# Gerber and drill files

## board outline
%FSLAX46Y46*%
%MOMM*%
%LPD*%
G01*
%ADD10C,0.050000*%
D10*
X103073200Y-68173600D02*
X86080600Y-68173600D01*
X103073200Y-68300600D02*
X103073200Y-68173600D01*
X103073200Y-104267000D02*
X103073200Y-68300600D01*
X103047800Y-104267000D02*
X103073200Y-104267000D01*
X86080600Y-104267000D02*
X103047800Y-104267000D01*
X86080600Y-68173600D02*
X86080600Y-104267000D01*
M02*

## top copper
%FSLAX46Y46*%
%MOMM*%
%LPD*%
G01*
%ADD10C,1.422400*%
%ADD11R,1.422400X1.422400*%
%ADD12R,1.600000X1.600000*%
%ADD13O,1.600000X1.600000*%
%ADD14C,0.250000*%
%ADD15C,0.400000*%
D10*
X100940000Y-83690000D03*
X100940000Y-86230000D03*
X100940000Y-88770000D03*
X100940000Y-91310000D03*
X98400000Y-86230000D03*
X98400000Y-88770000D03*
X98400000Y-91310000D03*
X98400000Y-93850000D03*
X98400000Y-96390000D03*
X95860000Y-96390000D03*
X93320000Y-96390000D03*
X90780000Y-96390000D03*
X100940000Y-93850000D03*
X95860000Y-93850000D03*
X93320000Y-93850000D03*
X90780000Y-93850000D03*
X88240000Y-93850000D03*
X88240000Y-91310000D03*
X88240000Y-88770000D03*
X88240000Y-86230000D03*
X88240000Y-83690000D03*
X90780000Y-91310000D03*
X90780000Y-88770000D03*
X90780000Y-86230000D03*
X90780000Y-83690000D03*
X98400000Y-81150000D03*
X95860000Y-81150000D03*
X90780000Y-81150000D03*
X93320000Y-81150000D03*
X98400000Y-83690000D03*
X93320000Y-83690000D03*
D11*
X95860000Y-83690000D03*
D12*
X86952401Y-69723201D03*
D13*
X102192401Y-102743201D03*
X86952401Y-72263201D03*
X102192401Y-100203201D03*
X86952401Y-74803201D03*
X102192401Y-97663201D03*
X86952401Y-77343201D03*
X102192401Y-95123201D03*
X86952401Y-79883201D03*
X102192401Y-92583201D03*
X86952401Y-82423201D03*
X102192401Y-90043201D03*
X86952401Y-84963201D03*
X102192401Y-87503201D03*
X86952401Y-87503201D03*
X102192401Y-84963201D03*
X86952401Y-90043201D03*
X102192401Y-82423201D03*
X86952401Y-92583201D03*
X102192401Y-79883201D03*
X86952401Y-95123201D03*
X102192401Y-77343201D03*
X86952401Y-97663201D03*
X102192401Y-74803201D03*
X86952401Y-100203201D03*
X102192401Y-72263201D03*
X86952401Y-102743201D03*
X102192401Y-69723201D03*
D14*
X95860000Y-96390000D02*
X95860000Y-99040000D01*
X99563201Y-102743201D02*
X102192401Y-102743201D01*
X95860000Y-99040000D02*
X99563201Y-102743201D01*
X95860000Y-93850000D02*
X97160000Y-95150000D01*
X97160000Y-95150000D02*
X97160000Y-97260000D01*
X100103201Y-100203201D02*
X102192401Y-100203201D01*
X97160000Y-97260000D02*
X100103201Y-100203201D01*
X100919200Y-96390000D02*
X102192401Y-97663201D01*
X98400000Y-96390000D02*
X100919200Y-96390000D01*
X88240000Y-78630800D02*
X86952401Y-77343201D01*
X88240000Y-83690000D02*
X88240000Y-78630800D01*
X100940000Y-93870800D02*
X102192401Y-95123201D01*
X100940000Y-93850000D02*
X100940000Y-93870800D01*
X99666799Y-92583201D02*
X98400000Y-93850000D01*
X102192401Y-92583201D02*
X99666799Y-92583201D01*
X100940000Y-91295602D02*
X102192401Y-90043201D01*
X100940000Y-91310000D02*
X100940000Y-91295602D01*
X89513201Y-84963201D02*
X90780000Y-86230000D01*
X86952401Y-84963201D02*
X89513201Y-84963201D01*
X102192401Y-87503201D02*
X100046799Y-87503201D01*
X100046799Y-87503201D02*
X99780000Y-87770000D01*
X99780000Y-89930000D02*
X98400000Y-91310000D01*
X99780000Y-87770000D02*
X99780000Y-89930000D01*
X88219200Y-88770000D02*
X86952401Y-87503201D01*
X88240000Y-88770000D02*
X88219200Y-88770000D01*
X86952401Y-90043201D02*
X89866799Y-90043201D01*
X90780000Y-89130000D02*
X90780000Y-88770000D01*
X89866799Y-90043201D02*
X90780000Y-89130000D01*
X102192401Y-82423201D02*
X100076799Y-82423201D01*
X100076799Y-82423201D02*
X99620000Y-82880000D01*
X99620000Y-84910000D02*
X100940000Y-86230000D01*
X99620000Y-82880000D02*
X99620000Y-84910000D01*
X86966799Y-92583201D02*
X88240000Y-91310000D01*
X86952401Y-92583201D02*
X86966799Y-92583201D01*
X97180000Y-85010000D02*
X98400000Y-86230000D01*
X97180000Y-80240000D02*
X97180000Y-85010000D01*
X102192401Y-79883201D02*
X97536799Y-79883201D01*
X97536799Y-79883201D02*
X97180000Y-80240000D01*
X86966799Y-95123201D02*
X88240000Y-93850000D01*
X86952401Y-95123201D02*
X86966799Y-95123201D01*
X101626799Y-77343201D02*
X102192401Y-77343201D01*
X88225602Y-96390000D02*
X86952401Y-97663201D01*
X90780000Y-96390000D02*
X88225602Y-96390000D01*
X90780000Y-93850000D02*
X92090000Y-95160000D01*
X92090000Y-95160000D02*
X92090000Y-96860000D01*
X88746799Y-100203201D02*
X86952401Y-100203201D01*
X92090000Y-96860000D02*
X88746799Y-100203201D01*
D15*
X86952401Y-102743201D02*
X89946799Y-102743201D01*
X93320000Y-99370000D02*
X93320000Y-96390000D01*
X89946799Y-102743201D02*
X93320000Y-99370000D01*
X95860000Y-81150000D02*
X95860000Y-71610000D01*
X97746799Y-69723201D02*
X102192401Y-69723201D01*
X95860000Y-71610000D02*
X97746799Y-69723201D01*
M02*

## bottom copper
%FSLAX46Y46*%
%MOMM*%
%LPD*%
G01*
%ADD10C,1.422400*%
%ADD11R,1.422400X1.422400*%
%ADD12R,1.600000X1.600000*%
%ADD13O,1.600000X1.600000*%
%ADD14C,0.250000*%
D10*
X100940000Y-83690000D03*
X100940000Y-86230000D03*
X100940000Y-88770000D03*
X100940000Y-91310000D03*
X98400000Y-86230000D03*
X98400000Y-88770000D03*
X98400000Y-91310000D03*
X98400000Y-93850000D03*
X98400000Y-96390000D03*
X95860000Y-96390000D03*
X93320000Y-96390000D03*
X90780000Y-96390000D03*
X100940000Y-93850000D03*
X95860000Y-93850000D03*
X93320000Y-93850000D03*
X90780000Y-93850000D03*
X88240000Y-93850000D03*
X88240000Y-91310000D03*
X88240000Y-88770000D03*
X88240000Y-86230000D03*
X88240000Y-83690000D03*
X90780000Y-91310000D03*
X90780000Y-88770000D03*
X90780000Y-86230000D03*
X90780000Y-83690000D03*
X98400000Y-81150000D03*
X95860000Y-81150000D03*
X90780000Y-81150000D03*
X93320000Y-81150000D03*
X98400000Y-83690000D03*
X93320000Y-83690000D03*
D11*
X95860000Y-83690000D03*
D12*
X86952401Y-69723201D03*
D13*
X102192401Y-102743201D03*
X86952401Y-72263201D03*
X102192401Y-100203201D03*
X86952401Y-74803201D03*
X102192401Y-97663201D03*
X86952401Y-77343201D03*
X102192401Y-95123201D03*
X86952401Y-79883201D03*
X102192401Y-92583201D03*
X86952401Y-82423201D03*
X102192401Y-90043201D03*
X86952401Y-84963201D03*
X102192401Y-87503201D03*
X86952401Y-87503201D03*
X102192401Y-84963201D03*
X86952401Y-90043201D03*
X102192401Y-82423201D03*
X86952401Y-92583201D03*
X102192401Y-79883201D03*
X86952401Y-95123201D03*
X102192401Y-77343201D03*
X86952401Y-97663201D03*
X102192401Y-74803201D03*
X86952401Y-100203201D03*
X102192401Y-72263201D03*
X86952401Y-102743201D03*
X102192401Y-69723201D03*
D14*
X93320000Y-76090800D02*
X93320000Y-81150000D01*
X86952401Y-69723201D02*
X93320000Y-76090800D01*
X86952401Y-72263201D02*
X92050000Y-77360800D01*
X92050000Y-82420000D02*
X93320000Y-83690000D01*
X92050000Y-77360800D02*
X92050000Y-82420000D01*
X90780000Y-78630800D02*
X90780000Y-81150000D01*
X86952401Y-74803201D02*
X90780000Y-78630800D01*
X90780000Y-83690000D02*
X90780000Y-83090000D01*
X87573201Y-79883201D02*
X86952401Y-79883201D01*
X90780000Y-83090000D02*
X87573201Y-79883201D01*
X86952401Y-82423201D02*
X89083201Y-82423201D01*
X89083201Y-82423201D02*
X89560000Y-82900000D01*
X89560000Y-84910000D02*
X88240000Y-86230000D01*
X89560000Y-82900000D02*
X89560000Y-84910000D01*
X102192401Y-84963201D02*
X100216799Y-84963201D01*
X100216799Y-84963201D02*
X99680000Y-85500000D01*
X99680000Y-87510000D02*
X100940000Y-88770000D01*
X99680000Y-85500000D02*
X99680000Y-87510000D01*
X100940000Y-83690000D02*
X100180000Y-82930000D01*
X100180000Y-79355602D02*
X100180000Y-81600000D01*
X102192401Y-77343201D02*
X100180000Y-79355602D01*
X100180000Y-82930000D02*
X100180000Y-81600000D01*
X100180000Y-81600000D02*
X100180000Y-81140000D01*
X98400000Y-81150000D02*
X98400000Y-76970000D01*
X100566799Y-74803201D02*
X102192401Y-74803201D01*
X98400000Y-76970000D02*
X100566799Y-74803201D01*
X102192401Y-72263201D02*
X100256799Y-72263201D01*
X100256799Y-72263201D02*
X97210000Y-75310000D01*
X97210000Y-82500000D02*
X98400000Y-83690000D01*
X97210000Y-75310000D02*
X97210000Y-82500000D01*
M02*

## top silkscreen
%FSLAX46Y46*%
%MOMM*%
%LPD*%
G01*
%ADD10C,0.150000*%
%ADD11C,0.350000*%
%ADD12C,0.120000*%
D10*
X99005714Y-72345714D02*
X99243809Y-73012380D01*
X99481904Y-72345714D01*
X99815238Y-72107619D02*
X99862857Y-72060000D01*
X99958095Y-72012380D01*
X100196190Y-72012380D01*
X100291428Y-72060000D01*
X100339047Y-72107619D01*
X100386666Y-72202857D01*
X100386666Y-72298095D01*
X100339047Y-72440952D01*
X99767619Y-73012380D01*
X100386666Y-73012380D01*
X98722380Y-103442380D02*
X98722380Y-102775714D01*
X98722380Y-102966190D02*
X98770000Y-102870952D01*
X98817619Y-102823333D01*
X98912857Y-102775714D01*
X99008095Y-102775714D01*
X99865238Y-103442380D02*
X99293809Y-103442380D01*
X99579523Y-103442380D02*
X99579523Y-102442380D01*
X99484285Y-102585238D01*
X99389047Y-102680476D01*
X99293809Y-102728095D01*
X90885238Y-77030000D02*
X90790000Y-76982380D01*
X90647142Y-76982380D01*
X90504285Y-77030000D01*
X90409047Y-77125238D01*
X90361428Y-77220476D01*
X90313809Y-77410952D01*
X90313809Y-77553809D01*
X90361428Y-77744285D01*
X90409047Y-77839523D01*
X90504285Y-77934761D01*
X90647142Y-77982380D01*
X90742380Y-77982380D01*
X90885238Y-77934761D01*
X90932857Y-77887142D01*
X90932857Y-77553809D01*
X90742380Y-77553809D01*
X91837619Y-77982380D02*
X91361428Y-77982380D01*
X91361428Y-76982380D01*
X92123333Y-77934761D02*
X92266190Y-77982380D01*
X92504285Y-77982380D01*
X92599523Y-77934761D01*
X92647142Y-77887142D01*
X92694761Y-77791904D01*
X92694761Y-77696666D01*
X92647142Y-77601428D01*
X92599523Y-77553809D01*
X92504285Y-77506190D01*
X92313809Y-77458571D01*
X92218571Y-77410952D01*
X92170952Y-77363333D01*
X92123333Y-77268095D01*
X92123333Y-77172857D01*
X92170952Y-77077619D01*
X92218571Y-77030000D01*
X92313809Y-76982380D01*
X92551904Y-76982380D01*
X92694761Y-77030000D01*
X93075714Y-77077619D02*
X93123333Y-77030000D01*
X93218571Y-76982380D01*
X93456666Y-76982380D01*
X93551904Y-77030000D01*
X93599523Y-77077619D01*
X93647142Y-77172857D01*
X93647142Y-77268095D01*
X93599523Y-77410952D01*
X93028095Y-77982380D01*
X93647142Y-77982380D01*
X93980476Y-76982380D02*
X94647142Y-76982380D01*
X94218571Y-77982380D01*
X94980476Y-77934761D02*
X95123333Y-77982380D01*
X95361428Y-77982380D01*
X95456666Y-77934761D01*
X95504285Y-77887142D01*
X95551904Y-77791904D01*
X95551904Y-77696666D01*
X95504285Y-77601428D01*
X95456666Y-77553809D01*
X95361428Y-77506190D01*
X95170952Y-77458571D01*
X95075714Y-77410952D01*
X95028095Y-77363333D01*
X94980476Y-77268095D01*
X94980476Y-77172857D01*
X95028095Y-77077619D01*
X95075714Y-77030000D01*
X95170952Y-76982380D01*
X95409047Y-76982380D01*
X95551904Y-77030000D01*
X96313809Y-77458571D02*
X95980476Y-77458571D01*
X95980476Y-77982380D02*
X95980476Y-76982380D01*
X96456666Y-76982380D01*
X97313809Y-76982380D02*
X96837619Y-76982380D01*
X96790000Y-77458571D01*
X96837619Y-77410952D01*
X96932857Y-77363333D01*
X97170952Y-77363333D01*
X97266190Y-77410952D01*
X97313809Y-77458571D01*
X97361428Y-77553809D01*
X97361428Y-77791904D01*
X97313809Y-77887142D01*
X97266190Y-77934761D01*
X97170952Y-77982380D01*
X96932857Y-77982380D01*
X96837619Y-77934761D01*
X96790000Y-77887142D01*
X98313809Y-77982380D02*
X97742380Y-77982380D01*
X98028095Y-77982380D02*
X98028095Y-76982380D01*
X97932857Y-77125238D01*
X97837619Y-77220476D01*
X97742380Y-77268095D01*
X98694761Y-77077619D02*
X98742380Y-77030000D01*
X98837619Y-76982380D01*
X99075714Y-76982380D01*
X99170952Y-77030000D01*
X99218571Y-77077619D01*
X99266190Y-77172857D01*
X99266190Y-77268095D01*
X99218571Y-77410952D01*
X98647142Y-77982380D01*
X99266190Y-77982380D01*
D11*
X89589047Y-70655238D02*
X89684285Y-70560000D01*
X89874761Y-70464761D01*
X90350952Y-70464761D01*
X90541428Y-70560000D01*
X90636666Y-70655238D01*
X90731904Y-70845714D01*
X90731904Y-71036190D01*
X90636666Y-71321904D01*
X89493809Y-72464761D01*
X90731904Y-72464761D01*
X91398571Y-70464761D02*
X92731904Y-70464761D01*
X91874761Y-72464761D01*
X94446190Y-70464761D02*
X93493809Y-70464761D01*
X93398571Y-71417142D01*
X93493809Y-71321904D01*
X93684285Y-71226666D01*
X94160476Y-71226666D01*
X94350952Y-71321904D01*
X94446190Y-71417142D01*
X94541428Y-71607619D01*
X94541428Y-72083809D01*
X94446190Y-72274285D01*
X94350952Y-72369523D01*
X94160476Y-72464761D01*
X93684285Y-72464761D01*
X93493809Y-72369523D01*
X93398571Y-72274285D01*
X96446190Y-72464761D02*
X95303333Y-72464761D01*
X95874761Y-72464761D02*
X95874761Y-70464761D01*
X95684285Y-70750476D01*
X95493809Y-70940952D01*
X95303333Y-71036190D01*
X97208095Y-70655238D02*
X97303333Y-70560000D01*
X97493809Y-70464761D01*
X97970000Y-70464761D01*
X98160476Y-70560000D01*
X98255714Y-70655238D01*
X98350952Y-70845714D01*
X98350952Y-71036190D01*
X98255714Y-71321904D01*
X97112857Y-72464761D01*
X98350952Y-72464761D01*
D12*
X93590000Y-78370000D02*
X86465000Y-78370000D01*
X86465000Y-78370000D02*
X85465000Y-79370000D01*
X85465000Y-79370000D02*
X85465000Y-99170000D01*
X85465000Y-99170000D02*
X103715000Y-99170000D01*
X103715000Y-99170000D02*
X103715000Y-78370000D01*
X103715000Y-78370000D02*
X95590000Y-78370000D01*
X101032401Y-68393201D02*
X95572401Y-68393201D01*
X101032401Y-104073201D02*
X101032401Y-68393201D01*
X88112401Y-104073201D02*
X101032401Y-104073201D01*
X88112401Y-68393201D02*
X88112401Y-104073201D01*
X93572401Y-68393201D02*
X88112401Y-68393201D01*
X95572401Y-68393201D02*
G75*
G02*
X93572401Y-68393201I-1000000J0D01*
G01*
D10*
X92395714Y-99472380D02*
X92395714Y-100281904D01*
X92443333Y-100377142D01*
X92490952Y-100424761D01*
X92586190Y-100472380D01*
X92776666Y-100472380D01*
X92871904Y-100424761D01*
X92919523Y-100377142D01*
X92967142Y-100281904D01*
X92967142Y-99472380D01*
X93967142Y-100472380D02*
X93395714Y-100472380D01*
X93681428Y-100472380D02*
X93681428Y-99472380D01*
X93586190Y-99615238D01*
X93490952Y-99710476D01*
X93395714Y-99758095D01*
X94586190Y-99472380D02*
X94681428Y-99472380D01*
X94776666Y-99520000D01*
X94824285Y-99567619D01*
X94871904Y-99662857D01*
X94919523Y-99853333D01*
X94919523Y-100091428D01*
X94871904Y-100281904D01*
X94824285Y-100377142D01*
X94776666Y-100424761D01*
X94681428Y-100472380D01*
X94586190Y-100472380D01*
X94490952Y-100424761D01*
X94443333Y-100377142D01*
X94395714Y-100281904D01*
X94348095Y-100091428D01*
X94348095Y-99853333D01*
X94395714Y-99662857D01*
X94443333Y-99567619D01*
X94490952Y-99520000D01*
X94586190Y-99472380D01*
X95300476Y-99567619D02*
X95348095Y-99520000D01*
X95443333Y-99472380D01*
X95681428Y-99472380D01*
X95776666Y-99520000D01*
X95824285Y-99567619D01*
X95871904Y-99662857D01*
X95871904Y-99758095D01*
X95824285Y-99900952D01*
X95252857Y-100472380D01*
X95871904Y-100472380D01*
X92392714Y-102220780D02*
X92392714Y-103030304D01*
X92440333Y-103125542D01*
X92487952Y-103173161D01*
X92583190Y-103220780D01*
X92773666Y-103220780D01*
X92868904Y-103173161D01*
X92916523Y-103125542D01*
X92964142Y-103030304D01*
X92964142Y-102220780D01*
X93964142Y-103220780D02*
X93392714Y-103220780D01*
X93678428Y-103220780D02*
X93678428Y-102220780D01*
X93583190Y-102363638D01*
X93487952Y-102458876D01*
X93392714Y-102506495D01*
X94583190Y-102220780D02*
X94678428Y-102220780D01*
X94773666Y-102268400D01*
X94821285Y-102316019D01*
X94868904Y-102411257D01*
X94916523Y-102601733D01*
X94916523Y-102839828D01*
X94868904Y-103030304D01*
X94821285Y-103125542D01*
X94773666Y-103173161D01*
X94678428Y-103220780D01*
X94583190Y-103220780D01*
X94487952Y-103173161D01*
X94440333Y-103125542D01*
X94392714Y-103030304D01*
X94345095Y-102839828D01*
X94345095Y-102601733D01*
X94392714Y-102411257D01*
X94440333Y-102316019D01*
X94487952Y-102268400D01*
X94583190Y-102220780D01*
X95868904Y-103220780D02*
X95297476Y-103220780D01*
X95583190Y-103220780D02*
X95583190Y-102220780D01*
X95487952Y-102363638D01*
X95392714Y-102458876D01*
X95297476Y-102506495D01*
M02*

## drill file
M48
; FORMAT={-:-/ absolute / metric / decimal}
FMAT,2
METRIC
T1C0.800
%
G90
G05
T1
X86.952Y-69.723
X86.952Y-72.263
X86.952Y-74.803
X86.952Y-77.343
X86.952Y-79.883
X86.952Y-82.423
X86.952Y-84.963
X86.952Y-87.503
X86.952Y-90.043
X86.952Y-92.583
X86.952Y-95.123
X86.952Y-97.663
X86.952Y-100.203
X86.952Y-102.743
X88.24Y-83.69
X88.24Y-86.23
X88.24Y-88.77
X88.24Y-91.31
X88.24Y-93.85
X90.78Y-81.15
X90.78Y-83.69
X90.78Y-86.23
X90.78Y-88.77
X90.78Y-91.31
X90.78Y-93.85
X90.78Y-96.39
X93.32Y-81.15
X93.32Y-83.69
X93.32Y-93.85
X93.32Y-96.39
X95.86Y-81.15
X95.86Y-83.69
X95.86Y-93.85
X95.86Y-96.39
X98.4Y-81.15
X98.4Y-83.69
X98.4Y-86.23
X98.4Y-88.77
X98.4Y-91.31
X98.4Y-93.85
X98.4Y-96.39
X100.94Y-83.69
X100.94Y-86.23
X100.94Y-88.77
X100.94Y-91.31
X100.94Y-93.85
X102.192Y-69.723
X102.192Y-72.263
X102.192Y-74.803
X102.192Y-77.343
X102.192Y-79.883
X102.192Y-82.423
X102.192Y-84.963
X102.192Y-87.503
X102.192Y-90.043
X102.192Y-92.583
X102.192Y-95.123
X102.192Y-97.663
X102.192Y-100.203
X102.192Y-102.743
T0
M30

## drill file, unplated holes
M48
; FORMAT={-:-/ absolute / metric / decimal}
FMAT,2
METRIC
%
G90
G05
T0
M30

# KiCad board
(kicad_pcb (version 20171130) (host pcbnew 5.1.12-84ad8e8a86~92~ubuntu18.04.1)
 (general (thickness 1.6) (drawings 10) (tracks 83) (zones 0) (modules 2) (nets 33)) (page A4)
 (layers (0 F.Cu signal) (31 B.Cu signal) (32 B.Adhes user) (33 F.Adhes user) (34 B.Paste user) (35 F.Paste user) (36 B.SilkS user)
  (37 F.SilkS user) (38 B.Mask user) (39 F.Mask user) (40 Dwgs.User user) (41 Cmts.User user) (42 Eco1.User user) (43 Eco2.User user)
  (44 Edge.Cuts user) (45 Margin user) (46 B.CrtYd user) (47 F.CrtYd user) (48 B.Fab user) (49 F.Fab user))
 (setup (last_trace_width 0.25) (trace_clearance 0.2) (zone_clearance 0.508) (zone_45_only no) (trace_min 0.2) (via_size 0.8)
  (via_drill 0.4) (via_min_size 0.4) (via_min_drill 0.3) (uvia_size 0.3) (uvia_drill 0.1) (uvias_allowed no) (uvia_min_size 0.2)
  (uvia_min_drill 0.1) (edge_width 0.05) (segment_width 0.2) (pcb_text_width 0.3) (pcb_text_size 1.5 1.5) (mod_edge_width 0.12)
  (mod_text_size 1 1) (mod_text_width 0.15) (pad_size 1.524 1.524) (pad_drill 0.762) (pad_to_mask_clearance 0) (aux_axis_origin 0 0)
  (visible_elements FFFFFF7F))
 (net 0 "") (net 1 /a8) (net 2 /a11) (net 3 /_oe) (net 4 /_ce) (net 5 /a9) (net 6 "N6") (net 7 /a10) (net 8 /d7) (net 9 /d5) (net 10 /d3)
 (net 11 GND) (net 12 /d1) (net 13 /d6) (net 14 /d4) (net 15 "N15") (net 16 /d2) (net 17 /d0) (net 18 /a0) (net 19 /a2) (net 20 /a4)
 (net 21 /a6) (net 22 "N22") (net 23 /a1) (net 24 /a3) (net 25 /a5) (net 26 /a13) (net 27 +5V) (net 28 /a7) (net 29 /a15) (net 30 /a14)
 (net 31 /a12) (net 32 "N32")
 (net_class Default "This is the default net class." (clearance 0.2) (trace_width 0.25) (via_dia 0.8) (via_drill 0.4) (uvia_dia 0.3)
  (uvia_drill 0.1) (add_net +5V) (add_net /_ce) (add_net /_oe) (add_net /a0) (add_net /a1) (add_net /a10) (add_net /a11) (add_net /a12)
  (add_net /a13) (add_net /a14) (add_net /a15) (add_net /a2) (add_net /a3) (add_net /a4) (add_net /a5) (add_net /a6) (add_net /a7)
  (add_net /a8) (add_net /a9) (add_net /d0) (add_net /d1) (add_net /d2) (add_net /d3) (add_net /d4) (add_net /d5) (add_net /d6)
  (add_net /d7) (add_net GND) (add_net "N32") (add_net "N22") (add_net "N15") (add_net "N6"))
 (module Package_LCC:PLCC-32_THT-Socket (layer F.Cu) (at 95.86 83.69)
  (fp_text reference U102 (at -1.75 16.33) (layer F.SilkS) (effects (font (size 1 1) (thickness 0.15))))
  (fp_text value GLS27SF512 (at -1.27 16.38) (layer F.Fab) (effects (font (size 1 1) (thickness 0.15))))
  (fp_line (start -2.27 -5.32) (end -9.395 -5.32) (layer F.SilkS) (width 0.12))
  (fp_line (start -9.395 -5.32) (end -10.395 -4.32) (layer F.SilkS) (width 0.12))
  (fp_line (start -10.395 -4.32) (end -10.395 15.48) (layer F.SilkS) (width 0.12))
  (fp_line (start -10.395 15.48) (end 7.855 15.48) (layer F.SilkS) (width 0.12))
  (fp_line (start 7.855 15.48) (end 7.855 -5.32) (layer F.SilkS) (width 0.12))
  (fp_line (start 7.855 -5.32) (end -0.27 -5.32) (layer F.SilkS) (width 0.12))
  (pad 29 thru_hole circle (at 5.08 0) (size 1.4224 1.4224) (drill 0.8) (layers *.Cu *.Mask) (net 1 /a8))
  (pad 27 thru_hole circle (at 5.08 2.54) (size 1.4224 1.4224) (drill 0.8) (layers *.Cu *.Mask) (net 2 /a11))
  (pad 25 thru_hole circle (at 5.08 5.08) (size 1.4224 1.4224) (drill 0.8) (layers *.Cu *.Mask) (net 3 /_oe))
  (pad 23 thru_hole circle (at 5.08 7.62) (size 1.4224 1.4224) (drill 0.8) (layers *.Cu *.Mask) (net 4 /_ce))
  (pad 28 thru_hole circle (at 2.54 2.54) (size 1.4224 1.4224) (drill 0.8) (layers *.Cu *.Mask) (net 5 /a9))
  (pad 26 thru_hole circle (at 2.54 5.08) (size 1.4224 1.4224) (drill 0.8) (layers *.Cu *.Mask) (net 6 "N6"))
  (pad 24 thru_hole circle (at 2.54 7.62) (size 1.4224 1.4224) (drill 0.8) (layers *.Cu *.Mask) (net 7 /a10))
  (pad 22 thru_hole circle (at 2.54 10.16) (size 1.4224 1.4224) (drill 0.8) (layers *.Cu *.Mask) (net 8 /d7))
  (pad 20 thru_hole circle (at 2.54 12.7) (size 1.4224 1.4224) (drill 0.8) (layers *.Cu *.Mask) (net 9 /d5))
  (pad 18 thru_hole circle (at 0 12.7) (size 1.4224 1.4224) (drill 0.8) (layers *.Cu *.Mask) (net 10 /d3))
  (pad 16 thru_hole circle (at -2.54 12.7) (size 1.4224 1.4224) (drill 0.8) (layers *.Cu *.Mask) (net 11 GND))
  (pad 14 thru_hole circle (at -5.08 12.7) (size 1.4224 1.4224) (drill 0.8) (layers *.Cu *.Mask) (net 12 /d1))
  (pad 21 thru_hole circle (at 5.08 10.16) (size 1.4224 1.4224) (drill 0.8) (layers *.Cu *.Mask) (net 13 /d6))
  (pad 19 thru_hole circle (at 0 10.16) (size 1.4224 1.4224) (drill 0.8) (layers *.Cu *.Mask) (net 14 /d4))
  (pad 17 thru_hole circle (at -2.54 10.16) (size 1.4224 1.4224) (drill 0.8) (layers *.Cu *.Mask) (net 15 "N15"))
  (pad 15 thru_hole circle (at -5.08 10.16) (size 1.4224 1.4224) (drill 0.8) (layers *.Cu *.Mask) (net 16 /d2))
  (pad 13 thru_hole circle (at -7.62 10.16) (size 1.4224 1.4224) (drill 0.8) (layers *.Cu *.Mask) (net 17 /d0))
  (pad 11 thru_hole circle (at -7.62 7.62) (size 1.4224 1.4224) (drill 0.8) (layers *.Cu *.Mask) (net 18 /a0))
  (pad 9 thru_hole circle (at -7.62 5.08) (size 1.4224 1.4224) (drill 0.8) (layers *.Cu *.Mask) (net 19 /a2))
  (pad 7 thru_hole circle (at -7.62 2.54) (size 1.4224 1.4224) (drill 0.8) (layers *.Cu *.Mask) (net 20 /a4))
  (pad 5 thru_hole circle (at -7.62 0) (size 1.4224 1.4224) (drill 0.8) (layers *.Cu *.Mask) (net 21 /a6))
  (pad 12 thru_hole circle (at -5.08 7.62) (size 1.4224 1.4224) (drill 0.8) (layers *.Cu *.Mask) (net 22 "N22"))
  (pad 10 thru_hole circle (at -5.08 5.08) (size 1.4224 1.4224) (drill 0.8) (layers *.Cu *.Mask) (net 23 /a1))
  (pad 8 thru_hole circle (at -5.08 2.54) (size 1.4224 1.4224) (drill 0.8) (layers *.Cu *.Mask) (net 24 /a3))
  (pad 6 thru_hole circle (at -5.08 0) (size 1.4224 1.4224) (drill 0.8) (layers *.Cu *.Mask) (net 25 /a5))
  (pad 30 thru_hole circle (at 2.54 -2.54) (size 1.4224 1.4224) (drill 0.8) (layers *.Cu *.Mask) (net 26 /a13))
  (pad 32 thru_hole circle (at 0 -2.54) (size 1.4224 1.4224) (drill 0.8) (layers *.Cu *.Mask) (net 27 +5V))
  (pad 4 thru_hole circle (at -5.08 -2.54) (size 1.4224 1.4224) (drill 0.8) (layers *.Cu *.Mask) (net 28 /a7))
  (pad 2 thru_hole circle (at -2.54 -2.54) (size 1.4224 1.4224) (drill 0.8) (layers *.Cu *.Mask) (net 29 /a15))
  (pad 31 thru_hole circle (at 2.54 0) (size 1.4224 1.4224) (drill 0.8) (layers *.Cu *.Mask) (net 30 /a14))
  (pad 3 thru_hole circle (at -2.54 0) (size 1.4224 1.4224) (drill 0.8) (layers *.Cu *.Mask) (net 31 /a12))
  (pad 1 thru_hole rect (at 0 0) (size 1.4224 1.4224) (drill 0.8) (layers *.Cu *.Mask) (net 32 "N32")))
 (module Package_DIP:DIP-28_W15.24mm (layer F.Cu) (at 86.952401 69.723201)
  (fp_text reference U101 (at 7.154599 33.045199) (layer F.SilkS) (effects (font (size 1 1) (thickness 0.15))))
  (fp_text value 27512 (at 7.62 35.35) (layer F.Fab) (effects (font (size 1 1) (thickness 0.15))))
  (fp_line (start 14.08 -1.33) (end 8.62 -1.33) (layer F.SilkS) (width 0.12))
  (fp_line (start 14.08 34.35) (end 14.08 -1.33) (layer F.SilkS) (width 0.12))
  (fp_line (start 1.16 34.35) (end 14.08 34.35) (layer F.SilkS) (width 0.12))
  (fp_line (start 1.16 -1.33) (end 1.16 34.35) (layer F.SilkS) (width 0.12))
  (fp_line (start 6.62 -1.33) (end 1.16 -1.33) (layer F.SilkS) (width 0.12))
  (fp_arc (start 7.62 -1.33) (end 6.62 -1.33) (angle -180) (layer F.SilkS) (width 0.12))
  (pad 1 thru_hole rect (at 0 0) (size 1.6 1.6) (drill 0.8) (layers *.Cu *.Mask) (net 29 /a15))
  (pad 15 thru_hole oval (at 15.24 33.02) (size 1.6 1.6) (drill 0.8) (layers *.Cu *.Mask) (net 10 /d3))
  (pad 2 thru_hole oval (at 0 2.54) (size 1.6 1.6) (drill 0.8) (layers *.Cu *.Mask) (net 31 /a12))
  (pad 16 thru_hole oval (at 15.24 30.48) (size 1.6 1.6) (drill 0.8) (layers *.Cu *.Mask) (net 14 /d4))
  (pad 3 thru_hole oval (at 0 5.08) (size 1.6 1.6) (drill 0.8) (layers *.Cu *.Mask) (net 28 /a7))
  (pad 17 thru_hole oval (at 15.24 27.94) (size 1.6 1.6) (drill 0.8) (layers *.Cu *.Mask) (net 9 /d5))
  (pad 4 thru_hole oval (at 0 7.62) (size 1.6 1.6) (drill 0.8) (layers *.Cu *.Mask) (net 21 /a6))
  (pad 18 thru_hole oval (at 15.24 25.4) (size 1.6 1.6) (drill 0.8) (layers *.Cu *.Mask) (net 13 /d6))
  (pad 5 thru_hole oval (at 0 10.16) (size 1.6 1.6) (drill 0.8) (layers *.Cu *.Mask) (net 25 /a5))
  (pad 19 thru_hole oval (at 15.24 22.86) (size 1.6 1.6) (drill 0.8) (layers *.Cu *.Mask) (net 8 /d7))
  (pad 6 thru_hole oval (at 0 12.7) (size 1.6 1.6) (drill 0.8) (layers *.Cu *.Mask) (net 20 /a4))
  (pad 20 thru_hole oval (at 15.24 20.32) (size 1.6 1.6) (drill 0.8) (layers *.Cu *.Mask) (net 4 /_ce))
  (pad 7 thru_hole oval (at 0 15.24) (size 1.6 1.6) (drill 0.8) (layers *.Cu *.Mask) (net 24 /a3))
  (pad 21 thru_hole oval (at 15.24 17.78) (size 1.6 1.6) (drill 0.8) (layers *.Cu *.Mask) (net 7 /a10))
  (pad 8 thru_hole oval (at 0 17.78) (size 1.6 1.6) (drill 0.8) (layers *.Cu *.Mask) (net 19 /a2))
  (pad 22 thru_hole oval (at 15.24 15.24) (size 1.6 1.6) (drill 0.8) (layers *.Cu *.Mask) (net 3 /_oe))
  (pad 9 thru_hole oval (at 0 20.32) (size 1.6 1.6) (drill 0.8) (layers *.Cu *.Mask) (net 23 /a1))
  (pad 23 thru_hole oval (at 15.24 12.7) (size 1.6 1.6) (drill 0.8) (layers *.Cu *.Mask) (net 2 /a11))
  (pad 10 thru_hole oval (at 0 22.86) (size 1.6 1.6) (drill 0.8) (layers *.Cu *.Mask) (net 18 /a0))
  (pad 24 thru_hole oval (at 15.24 10.16) (size 1.6 1.6) (drill 0.8) (layers *.Cu *.Mask) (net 5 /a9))
  (pad 11 thru_hole oval (at 0 25.4) (size 1.6 1.6) (drill 0.8) (layers *.Cu *.Mask) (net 17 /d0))
  (pad 25 thru_hole oval (at 15.24 7.62) (size 1.6 1.6) (drill 0.8) (layers *.Cu *.Mask) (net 1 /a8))
  (pad 12 thru_hole oval (at 0 27.94) (size 1.6 1.6) (drill 0.8) (layers *.Cu *.Mask) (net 12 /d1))
  (pad 26 thru_hole oval (at 15.24 5.08) (size 1.6 1.6) (drill 0.8) (layers *.Cu *.Mask) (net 26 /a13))
  (pad 13 thru_hole oval (at 0 30.48) (size 1.6 1.6) (drill 0.8) (layers *.Cu *.Mask) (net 16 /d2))
  (pad 27 thru_hole oval (at 15.24 2.54) (size 1.6 1.6) (drill 0.8) (layers *.Cu *.Mask) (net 30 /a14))
  (pad 14 thru_hole oval (at 0 33.02) (size 1.6 1.6) (drill 0.8) (layers *.Cu *.Mask) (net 11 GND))
  (pad 28 thru_hole oval (at 15.24 0) (size 1.6 1.6) (drill 0.8) (layers *.Cu *.Mask) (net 27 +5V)))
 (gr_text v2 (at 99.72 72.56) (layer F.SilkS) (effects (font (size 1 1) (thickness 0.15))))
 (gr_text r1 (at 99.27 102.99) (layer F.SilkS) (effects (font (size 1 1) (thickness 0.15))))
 (gr_line (start 103.0732 68.1736) (end 86.0806 68.1736) (layer Edge.Cuts) (width 0.05))
 (gr_line (start 103.0732 68.3006) (end 103.0732 68.1736) (layer Edge.Cuts) (width 0.05))
 (gr_line (start 103.0732 104.267) (end 103.0732 68.3006) (layer Edge.Cuts) (width 0.05))
 (gr_line (start 103.0478 104.267) (end 103.0732 104.267) (layer Edge.Cuts) (width 0.05))
 (gr_line (start 86.0806 104.267) (end 103.0478 104.267) (layer Edge.Cuts) (width 0.05))
 (gr_line (start 86.0806 68.1736) (end 86.0806 104.267) (layer Edge.Cuts) (width 0.05))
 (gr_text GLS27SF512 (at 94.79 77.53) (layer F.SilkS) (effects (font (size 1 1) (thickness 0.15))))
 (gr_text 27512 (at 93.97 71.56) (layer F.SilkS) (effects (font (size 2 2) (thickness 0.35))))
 (segment (start 93.32 76.0908) (end 93.32 81.15) (width 0.25) (layer B.Cu) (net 29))
 (segment (start 86.952401 69.723201) (end 93.32 76.0908) (width 0.25) (layer B.Cu) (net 29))
 (segment (start 95.86 96.39) (end 95.86 99.04) (width 0.25) (layer F.Cu) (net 10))
 (segment (start 99.563201 102.743201) (end 102.192401 102.743201) (width 0.25) (layer F.Cu) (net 10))
 (segment (start 95.86 99.04) (end 99.563201 102.743201) (width 0.25) (layer F.Cu) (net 10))
 (segment (start 86.952401 72.263201) (end 92.05 77.3608) (width 0.25) (layer B.Cu) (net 31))
 (segment (start 92.05 82.42) (end 93.32 83.69) (width 0.25) (layer B.Cu) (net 31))
 (segment (start 92.05 77.3608) (end 92.05 82.42) (width 0.25) (layer B.Cu) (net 31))
 (segment (start 95.86 93.85) (end 97.16 95.15) (width 0.25) (layer F.Cu) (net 14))
 (segment (start 97.16 95.15) (end 97.16 97.26) (width 0.25) (layer F.Cu) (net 14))
 (segment (start 100.103201 100.203201) (end 102.192401 100.203201) (width 0.25) (layer F.Cu) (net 14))
 (segment (start 97.16 97.26) (end 100.103201 100.203201) (width 0.25) (layer F.Cu) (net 14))
 (segment (start 90.78 78.6308) (end 90.78 81.15) (width 0.25) (layer B.Cu) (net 28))
 (segment (start 86.952401 74.803201) (end 90.78 78.6308) (width 0.25) (layer B.Cu) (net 28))
 (segment (start 100.9192 96.39) (end 102.192401 97.663201) (width 0.25) (layer F.Cu) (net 9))
 (segment (start 98.4 96.39) (end 100.9192 96.39) (width 0.25) (layer F.Cu) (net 9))
 (segment (start 88.24 78.6308) (end 86.952401 77.343201) (width 0.25) (layer F.Cu) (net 21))
 (segment (start 88.24 83.69) (end 88.24 78.6308) (width 0.25) (layer F.Cu) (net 21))
 (segment (start 100.94 93.8708) (end 102.192401 95.123201) (width 0.25) (layer F.Cu) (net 13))
 (segment (start 100.94 93.85) (end 100.94 93.8708) (width 0.25) (layer F.Cu) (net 13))
 (segment (start 90.78 83.69) (end 90.78 83.09) (width 0.25) (layer B.Cu) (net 25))
 (segment (start 87.573201 79.883201) (end 86.952401 79.883201) (width 0.25) (layer B.Cu) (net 25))
 (segment (start 90.78 83.09) (end 87.573201 79.883201) (width 0.25) (layer B.Cu) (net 25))
 (segment (start 99.666799 92.583201) (end 98.4 93.85) (width 0.25) (layer F.Cu) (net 8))
 (segment (start 102.192401 92.583201) (end 99.666799 92.583201) (width 0.25) (layer F.Cu) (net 8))
 (segment (start 86.952401 82.423201) (end 89.083201 82.423201) (width 0.25) (layer B.Cu) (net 20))
 (segment (start 89.083201 82.423201) (end 89.56 82.9) (width 0.25) (layer B.Cu) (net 20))
 (segment (start 89.56 84.91) (end 88.24 86.23) (width 0.25) (layer B.Cu) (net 20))
 (segment (start 89.56 82.9) (end 89.56 84.91) (width 0.25) (layer B.Cu) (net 20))
 (segment (start 100.94 91.295602) (end 102.192401 90.043201) (width 0.25) (layer F.Cu) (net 4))
 (segment (start 100.94 91.31) (end 100.94 91.295602) (width 0.25) (layer F.Cu) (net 4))
 (segment (start 89.513201 84.963201) (end 90.78 86.23) (width 0.25) (layer F.Cu) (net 24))
 (segment (start 86.952401 84.963201) (end 89.513201 84.963201) (width 0.25) (layer F.Cu) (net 24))
 (segment (start 102.192401 87.503201) (end 100.046799 87.503201) (width 0.25) (layer F.Cu) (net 7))
 (segment (start 100.046799 87.503201) (end 99.78 87.77) (width 0.25) (layer F.Cu) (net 7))
 (segment (start 99.78 89.93) (end 98.4 91.31) (width 0.25) (layer F.Cu) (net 7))
 (segment (start 99.78 87.77) (end 99.78 89.93) (width 0.25) (layer F.Cu) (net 7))
 (segment (start 88.2192 88.77) (end 86.952401 87.503201) (width 0.25) (layer F.Cu) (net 19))
 (segment (start 88.24 88.77) (end 88.2192 88.77) (width 0.25) (layer F.Cu) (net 19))
 (segment (start 102.192401 84.963201) (end 100.216799 84.963201) (width 0.25) (layer B.Cu) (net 3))
 (segment (start 100.216799 84.963201) (end 99.68 85.5) (width 0.25) (layer B.Cu) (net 3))
 (segment (start 99.68 87.51) (end 100.94 88.77) (width 0.25) (layer B.Cu) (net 3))
 (segment (start 99.68 85.5) (end 99.68 87.51) (width 0.25) (layer B.Cu) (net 3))
 (segment (start 86.952401 90.043201) (end 89.866799 90.043201) (width 0.25) (layer F.Cu) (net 23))
 (segment (start 90.78 89.13) (end 90.78 88.77) (width 0.25) (layer F.Cu) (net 23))
 (segment (start 89.866799 90.043201) (end 90.78 89.13) (width 0.25) (layer F.Cu) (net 23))
 (segment (start 102.192401 82.423201) (end 100.076799 82.423201) (width 0.25) (layer F.Cu) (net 2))
 (segment (start 100.076799 82.423201) (end 99.62 82.88) (width 0.25) (layer F.Cu) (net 2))
 (segment (start 99.62 84.91) (end 100.94 86.23) (width 0.25) (layer F.Cu) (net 2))
 (segment (start 99.62 82.88) (end 99.62 84.91) (width 0.25) (layer F.Cu) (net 2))
 (segment (start 86.966799 92.583201) (end 88.24 91.31) (width 0.25) (layer F.Cu) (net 18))
 (segment (start 86.952401 92.583201) (end 86.966799 92.583201) (width 0.25) (layer F.Cu) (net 18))
 (segment (start 97.18 85.01) (end 98.4 86.23) (width 0.25) (layer F.Cu) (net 5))
 (segment (start 97.18 80.24) (end 97.18 85.01) (width 0.25) (layer F.Cu) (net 5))
 (segment (start 102.192401 79.883201) (end 97.536799 79.883201) (width 0.25) (layer F.Cu) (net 5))
 (segment (start 97.536799 79.883201) (end 97.18 80.24) (width 0.25) (layer F.Cu) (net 5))
 (segment (start 86.966799 95.123201) (end 88.24 93.85) (width 0.25) (layer F.Cu) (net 17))
 (segment (start 86.952401 95.123201) (end 86.966799 95.123201) (width 0.25) (layer F.Cu) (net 17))
 (segment (start 100.94 83.69) (end 100.18 82.93) (width 0.25) (layer B.Cu) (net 1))
 (segment (start 101.626799 77.343201) (end 102.192401 77.343201) (width 0.25) (layer F.Cu) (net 1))
 (segment (start 100.18 79.355602) (end 100.18 81.6) (width 0.25) (layer B.Cu) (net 1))
 (segment (start 102.192401 77.343201) (end 100.18 79.355602) (width 0.25) (layer B.Cu) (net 1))
 (segment (start 100.18 82.93) (end 100.18 81.6) (width 0.25) (layer B.Cu) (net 1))
 (segment (start 100.18 81.6) (end 100.18 81.14) (width 0.25) (layer B.Cu) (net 1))
 (segment (start 88.225602 96.39) (end 86.952401 97.663201) (width 0.25) (layer F.Cu) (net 12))
 (segment (start 90.78 96.39) (end 88.225602 96.39) (width 0.25) (layer F.Cu) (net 12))
 (segment (start 98.4 81.15) (end 98.4 76.97) (width 0.25) (layer B.Cu) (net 26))
 (segment (start 100.566799 74.803201) (end 102.192401 74.803201) (width 0.25) (layer B.Cu) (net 26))
 (segment (start 98.4 76.97) (end 100.566799 74.803201) (width 0.25) (layer B.Cu) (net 26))
 (segment (start 90.78 93.85) (end 92.09 95.16) (width 0.25) (layer F.Cu) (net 16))
 (segment (start 92.09 95.16) (end 92.09 96.86) (width 0.25) (layer F.Cu) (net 16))
 (segment (start 88.746799 100.203201) (end 86.952401 100.203201) (width 0.25) (layer F.Cu) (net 16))
 (segment (start 92.09 96.86) (end 88.746799 100.203201) (width 0.25) (layer F.Cu) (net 16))
 (segment (start 102.192401 72.263201) (end 100.256799 72.263201) (width 0.25) (layer B.Cu) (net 30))
 (segment (start 100.256799 72.263201) (end 97.21 75.31) (width 0.25) (layer B.Cu) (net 30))
 (segment (start 97.21 82.5) (end 98.4 83.69) (width 0.25) (layer B.Cu) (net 30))
 (segment (start 97.21 75.31) (end 97.21 82.5) (width 0.25) (layer B.Cu) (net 30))
 (segment (start 86.952401 102.743201) (end 89.946799 102.743201) (width 0.4) (layer F.Cu) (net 11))
 (segment (start 93.32 99.37) (end 93.32 96.39) (width 0.4) (layer F.Cu) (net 11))
 (segment (start 89.946799 102.743201) (end 93.32 99.37) (width 0.4) (layer F.Cu) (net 11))
 (segment (start 95.86 81.15) (end 95.86 71.61) (width 0.4) (layer F.Cu) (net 27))
 (segment (start 97.746799 69.723201) (end 102.192401 69.723201) (width 0.4) (layer F.Cu) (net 27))
 (segment (start 95.86 71.61) (end 97.746799 69.723201) (width 0.4) (layer F.Cu) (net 27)))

